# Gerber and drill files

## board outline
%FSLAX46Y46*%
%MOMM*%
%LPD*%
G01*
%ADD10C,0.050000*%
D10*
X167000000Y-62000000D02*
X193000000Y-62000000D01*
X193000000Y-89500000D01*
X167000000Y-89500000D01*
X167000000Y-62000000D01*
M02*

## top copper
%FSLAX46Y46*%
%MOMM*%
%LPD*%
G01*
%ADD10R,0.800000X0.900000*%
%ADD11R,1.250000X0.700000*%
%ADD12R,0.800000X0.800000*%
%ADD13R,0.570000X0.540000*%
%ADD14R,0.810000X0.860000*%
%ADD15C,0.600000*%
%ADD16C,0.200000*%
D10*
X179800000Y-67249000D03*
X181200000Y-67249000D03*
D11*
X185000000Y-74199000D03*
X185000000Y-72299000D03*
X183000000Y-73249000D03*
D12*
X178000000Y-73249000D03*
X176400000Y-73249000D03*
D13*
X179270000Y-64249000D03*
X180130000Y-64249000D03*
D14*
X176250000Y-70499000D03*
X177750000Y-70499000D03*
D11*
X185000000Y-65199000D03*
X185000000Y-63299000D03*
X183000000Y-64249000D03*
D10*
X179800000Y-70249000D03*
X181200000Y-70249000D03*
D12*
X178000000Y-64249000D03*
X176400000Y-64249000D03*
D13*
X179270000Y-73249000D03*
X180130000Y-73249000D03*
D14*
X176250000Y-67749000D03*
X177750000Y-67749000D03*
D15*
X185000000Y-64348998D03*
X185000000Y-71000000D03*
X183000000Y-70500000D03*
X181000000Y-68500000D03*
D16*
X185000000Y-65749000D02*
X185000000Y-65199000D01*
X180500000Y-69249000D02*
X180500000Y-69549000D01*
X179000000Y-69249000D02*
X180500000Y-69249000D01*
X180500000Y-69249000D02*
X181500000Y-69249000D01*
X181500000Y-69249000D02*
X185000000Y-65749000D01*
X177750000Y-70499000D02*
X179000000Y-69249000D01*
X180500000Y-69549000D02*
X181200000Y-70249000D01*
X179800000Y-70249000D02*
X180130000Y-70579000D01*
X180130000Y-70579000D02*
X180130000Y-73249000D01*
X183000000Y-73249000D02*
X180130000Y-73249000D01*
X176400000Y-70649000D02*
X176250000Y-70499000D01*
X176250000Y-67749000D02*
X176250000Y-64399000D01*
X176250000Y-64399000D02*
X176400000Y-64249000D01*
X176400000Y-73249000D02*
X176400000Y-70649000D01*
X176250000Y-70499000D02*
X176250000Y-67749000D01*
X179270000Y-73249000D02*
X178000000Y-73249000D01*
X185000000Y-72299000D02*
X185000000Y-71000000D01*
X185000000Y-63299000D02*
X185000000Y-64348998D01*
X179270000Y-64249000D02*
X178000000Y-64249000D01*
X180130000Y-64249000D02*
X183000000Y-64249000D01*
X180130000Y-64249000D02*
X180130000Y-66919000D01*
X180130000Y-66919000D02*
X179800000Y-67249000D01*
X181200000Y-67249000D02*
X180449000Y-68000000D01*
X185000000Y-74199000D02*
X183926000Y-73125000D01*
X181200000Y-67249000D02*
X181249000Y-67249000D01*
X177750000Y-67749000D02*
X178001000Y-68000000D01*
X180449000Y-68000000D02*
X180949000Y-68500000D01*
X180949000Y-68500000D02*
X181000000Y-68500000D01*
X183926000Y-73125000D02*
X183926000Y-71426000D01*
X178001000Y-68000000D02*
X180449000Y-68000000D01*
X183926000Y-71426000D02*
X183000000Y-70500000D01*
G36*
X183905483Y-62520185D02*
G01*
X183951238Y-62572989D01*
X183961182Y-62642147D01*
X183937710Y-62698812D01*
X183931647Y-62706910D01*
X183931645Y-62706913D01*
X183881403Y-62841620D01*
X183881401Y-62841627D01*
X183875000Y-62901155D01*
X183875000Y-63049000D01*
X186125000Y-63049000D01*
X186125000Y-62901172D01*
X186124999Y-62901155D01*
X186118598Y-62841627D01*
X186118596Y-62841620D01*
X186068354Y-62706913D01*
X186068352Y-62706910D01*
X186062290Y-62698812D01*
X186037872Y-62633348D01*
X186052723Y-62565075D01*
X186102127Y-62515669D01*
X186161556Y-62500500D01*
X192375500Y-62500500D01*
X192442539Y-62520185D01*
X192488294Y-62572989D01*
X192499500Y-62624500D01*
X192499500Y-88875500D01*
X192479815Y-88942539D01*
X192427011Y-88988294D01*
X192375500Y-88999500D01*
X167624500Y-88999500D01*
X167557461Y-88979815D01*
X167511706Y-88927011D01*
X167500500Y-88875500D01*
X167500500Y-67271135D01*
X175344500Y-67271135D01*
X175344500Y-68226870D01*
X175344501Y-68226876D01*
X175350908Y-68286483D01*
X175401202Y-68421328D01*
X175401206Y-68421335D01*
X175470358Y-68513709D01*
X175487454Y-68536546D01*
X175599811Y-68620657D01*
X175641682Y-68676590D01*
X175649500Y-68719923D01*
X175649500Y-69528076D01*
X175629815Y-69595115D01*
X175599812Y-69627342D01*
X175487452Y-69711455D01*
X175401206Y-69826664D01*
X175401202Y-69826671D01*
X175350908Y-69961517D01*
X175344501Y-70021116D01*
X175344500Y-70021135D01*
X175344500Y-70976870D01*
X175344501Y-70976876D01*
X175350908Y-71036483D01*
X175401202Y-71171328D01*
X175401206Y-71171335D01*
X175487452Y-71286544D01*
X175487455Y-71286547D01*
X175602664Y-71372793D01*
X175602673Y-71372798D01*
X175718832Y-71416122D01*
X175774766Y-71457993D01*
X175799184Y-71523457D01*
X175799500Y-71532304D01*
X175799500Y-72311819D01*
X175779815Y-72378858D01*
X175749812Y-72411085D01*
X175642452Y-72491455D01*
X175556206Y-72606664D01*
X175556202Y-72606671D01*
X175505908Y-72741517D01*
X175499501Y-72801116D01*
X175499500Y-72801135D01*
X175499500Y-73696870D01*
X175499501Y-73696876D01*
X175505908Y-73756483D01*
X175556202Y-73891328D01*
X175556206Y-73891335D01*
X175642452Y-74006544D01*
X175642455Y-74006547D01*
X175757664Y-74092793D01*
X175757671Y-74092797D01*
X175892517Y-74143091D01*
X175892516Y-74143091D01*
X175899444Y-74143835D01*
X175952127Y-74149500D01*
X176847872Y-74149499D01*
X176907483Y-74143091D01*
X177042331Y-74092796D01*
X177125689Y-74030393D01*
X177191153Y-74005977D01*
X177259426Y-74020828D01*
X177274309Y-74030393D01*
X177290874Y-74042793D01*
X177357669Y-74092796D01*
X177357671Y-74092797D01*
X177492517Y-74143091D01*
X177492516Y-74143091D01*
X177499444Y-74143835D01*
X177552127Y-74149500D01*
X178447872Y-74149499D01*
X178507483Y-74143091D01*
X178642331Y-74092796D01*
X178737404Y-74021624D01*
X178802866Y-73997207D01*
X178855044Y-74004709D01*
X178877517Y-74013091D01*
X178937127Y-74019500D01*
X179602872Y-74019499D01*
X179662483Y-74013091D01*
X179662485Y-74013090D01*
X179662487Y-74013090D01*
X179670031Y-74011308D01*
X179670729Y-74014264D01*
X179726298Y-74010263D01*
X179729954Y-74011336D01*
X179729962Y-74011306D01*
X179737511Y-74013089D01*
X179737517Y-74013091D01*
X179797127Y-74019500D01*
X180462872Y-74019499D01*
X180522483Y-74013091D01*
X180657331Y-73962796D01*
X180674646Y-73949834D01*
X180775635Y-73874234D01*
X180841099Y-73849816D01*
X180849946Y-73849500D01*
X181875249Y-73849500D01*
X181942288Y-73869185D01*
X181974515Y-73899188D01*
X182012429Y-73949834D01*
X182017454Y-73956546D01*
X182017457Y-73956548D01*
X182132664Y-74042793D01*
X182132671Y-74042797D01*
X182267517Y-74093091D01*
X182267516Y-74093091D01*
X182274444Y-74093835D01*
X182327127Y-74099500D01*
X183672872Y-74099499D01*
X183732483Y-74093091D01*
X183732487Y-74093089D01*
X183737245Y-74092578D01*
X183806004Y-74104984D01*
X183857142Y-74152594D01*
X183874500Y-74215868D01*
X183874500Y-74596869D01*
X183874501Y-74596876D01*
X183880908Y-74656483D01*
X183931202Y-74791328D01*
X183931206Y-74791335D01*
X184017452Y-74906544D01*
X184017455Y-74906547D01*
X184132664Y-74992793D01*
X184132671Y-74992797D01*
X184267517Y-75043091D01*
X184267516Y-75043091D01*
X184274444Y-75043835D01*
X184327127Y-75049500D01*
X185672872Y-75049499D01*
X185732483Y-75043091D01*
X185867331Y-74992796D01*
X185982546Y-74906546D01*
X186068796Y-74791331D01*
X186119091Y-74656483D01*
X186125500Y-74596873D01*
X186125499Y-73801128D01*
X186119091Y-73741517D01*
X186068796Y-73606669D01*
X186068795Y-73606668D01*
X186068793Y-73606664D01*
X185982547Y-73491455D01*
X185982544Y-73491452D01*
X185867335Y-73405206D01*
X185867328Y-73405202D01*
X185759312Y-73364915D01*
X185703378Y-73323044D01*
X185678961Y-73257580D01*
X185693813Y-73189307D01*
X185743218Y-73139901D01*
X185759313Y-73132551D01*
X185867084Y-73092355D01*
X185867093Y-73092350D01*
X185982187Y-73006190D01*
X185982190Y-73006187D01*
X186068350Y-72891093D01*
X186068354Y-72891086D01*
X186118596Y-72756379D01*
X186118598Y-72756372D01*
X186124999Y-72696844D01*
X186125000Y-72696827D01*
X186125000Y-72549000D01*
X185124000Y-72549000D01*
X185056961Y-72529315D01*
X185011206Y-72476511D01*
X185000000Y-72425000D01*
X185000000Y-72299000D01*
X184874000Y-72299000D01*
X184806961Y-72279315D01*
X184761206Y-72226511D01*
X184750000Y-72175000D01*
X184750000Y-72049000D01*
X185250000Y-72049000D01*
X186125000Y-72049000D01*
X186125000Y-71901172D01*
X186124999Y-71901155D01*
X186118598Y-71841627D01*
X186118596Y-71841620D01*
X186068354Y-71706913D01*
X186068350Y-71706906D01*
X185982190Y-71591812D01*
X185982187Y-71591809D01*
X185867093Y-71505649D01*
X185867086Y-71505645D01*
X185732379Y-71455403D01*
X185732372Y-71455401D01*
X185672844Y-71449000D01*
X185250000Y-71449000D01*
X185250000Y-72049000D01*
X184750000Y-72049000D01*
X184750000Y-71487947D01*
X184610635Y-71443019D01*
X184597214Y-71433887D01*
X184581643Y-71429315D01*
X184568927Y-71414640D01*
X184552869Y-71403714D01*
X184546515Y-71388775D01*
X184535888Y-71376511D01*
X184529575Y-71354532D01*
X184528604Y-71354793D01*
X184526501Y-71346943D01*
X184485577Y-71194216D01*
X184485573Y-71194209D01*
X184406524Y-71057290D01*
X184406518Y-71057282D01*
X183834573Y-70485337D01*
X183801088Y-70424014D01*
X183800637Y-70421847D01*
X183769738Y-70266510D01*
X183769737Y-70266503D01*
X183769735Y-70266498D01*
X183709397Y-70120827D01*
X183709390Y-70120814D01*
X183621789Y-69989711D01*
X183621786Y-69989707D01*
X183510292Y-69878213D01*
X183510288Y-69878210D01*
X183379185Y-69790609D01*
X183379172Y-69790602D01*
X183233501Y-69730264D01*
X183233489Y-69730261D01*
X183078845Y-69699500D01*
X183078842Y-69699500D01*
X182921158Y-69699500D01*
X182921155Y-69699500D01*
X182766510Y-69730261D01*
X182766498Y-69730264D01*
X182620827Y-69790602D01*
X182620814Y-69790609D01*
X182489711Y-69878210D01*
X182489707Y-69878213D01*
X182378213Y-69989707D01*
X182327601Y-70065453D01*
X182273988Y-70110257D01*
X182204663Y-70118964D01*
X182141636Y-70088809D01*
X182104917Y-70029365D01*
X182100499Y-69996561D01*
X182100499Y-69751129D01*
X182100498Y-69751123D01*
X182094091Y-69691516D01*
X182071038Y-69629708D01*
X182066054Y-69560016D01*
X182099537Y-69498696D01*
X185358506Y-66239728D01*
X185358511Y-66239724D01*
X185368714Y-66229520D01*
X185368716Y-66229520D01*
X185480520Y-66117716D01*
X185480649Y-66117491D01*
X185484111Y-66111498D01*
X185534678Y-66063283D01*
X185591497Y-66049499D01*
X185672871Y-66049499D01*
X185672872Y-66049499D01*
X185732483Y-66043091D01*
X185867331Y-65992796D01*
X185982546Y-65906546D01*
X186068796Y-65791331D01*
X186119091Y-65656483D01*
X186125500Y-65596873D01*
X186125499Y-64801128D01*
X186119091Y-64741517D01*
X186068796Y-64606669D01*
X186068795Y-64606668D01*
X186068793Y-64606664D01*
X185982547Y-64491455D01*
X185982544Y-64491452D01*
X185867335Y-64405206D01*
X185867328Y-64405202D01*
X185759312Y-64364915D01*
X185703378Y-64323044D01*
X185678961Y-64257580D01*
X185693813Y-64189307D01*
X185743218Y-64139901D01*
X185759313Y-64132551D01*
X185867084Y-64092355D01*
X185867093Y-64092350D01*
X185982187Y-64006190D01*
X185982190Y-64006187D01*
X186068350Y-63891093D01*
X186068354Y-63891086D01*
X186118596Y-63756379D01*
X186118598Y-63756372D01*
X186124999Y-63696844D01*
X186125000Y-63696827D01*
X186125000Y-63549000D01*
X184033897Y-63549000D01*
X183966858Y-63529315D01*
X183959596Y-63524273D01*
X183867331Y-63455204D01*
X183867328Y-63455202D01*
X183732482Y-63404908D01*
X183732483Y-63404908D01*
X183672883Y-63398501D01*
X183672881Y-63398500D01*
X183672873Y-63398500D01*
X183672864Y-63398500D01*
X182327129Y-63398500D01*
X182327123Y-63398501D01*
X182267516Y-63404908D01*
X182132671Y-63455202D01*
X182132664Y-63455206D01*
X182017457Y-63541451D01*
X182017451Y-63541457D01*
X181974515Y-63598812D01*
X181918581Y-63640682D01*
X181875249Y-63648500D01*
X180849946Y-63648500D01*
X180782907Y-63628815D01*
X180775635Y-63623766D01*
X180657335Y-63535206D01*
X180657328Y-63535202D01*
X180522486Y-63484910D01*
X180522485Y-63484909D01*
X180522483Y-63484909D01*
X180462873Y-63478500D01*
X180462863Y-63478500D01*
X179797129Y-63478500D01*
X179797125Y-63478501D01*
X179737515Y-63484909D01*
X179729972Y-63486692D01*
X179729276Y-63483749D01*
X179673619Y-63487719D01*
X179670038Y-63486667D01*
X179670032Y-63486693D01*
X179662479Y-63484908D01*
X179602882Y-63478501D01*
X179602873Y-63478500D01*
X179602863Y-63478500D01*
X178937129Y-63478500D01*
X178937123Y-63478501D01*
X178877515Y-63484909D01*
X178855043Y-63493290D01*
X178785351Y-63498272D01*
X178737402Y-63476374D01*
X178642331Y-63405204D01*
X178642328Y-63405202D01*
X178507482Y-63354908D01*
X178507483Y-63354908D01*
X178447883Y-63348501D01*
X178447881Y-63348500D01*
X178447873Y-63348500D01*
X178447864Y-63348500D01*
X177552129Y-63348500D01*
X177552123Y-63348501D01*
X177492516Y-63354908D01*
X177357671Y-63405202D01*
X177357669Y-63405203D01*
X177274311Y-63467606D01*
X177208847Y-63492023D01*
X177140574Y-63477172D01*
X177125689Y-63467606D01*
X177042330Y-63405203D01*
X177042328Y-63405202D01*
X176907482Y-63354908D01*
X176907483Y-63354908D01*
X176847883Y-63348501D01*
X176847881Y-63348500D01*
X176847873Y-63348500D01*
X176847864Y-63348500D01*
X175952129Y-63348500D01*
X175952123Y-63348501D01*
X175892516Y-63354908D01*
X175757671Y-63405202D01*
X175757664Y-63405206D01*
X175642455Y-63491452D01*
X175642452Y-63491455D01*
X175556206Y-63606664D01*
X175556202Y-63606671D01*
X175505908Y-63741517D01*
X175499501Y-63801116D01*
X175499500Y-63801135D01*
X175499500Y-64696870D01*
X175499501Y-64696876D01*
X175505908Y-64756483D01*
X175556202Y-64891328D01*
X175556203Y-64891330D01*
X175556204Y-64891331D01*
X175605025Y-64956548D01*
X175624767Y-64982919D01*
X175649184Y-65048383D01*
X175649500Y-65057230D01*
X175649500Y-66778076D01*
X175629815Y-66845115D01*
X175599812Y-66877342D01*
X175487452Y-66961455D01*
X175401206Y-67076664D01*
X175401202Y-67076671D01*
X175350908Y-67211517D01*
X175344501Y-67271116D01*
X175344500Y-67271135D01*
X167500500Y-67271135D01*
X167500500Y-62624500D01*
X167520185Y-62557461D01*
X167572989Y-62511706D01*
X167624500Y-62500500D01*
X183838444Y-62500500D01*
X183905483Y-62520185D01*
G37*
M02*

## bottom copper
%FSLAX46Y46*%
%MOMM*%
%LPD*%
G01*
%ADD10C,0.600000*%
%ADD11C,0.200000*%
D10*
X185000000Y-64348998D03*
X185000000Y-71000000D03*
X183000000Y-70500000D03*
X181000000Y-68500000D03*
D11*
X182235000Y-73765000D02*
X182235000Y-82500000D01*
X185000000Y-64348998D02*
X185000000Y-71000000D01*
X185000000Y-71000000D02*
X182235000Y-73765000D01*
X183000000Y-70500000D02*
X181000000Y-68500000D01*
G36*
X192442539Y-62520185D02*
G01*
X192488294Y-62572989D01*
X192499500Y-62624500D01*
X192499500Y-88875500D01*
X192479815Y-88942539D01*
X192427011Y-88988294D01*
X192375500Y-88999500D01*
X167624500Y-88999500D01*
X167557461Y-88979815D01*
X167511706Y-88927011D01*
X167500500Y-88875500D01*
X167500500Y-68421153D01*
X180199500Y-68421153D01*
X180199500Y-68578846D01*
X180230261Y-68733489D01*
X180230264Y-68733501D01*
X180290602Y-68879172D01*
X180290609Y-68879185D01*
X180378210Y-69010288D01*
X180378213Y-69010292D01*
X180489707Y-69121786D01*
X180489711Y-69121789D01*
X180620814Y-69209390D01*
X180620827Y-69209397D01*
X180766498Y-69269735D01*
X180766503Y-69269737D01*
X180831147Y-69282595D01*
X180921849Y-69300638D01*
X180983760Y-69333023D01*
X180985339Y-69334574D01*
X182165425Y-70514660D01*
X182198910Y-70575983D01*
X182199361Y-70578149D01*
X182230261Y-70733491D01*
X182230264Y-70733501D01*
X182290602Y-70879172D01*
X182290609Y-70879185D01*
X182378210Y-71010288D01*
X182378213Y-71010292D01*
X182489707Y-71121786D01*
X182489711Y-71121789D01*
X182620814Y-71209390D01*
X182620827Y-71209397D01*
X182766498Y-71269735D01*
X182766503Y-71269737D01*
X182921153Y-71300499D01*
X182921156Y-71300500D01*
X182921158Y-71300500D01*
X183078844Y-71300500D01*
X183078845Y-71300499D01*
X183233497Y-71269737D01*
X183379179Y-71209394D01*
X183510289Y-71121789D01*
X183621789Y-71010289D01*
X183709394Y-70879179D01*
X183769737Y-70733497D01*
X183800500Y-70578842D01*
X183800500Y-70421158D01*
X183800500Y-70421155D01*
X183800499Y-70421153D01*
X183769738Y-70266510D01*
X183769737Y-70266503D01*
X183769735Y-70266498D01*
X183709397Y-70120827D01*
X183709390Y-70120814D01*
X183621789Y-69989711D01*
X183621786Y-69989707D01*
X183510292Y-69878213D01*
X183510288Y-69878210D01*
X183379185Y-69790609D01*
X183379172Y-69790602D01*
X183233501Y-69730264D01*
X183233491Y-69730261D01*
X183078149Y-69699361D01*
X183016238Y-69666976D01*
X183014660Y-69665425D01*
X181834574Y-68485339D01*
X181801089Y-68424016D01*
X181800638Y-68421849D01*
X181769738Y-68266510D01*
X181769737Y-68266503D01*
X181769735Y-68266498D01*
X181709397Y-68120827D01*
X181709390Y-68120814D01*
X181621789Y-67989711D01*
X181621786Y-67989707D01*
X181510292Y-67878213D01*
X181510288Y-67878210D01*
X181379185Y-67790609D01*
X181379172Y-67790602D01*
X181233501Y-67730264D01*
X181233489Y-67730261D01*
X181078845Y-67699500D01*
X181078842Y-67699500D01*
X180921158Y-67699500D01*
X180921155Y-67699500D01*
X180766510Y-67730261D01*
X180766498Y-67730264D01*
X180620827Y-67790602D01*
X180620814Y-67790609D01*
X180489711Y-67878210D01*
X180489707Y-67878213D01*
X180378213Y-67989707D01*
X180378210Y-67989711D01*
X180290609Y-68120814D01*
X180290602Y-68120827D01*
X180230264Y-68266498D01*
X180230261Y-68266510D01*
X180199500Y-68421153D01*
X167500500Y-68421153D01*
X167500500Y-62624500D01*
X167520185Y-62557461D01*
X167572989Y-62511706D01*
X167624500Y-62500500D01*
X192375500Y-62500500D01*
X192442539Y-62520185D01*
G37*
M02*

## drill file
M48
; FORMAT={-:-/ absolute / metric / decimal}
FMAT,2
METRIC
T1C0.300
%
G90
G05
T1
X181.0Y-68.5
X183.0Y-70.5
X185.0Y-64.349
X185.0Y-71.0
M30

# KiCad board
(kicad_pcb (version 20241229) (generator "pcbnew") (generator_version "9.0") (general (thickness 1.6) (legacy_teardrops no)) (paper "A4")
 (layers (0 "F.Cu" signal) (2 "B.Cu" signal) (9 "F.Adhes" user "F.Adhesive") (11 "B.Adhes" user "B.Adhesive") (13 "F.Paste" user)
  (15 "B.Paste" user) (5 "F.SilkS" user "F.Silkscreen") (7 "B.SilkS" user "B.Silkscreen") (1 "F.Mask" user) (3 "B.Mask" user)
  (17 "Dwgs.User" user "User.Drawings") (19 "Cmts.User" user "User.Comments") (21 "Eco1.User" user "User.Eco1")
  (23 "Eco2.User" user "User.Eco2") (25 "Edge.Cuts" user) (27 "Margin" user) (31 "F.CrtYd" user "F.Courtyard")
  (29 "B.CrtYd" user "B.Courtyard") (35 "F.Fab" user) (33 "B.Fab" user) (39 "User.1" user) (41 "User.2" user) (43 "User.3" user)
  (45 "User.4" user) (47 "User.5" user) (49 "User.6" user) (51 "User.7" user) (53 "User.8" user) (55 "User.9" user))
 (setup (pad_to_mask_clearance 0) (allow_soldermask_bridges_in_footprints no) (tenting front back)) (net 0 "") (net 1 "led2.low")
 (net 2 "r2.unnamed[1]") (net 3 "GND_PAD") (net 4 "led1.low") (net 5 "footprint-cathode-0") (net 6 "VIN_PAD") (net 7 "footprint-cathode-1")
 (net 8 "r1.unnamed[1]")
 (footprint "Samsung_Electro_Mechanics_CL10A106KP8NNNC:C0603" (layer "F.Cu") (at 180.5 67.249 0)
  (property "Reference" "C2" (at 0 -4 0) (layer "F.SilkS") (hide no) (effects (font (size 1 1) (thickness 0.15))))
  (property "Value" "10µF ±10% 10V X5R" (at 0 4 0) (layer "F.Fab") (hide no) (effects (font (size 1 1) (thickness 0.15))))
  (pad "1" smd rect (at -0.7 0 0) (size 0.8 0.9) (layers "F.Cu" "F.Mask" "F.Paste") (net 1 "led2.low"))
  (pad "2" smd rect (at 0.7 0 0) (size 0.8 0.9) (layers "F.Cu" "F.Mask" "F.Paste") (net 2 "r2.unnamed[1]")))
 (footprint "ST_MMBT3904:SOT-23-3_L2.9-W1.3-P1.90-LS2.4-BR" (layer "F.Cu") (at 184 73.249 0)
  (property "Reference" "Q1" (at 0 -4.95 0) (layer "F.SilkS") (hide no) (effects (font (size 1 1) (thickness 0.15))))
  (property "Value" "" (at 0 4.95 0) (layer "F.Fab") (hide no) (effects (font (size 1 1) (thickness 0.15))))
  (pad "1" smd rect (at 1 0.95 0) (size 1.25 0.7) (layers "F.Cu" "F.Mask" "F.Paste") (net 2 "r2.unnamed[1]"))
  (pad "2" smd rect (at 1 -0.95 0) (size 1.25 0.7) (layers "F.Cu" "F.Mask" "F.Paste") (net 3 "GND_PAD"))
  (pad "3" smd rect (at -1 0 0) (size 1.25 0.7) (layers "F.Cu" "F.Mask" "F.Paste") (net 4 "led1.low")))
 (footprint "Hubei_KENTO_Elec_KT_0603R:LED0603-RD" (layer "F.Cu") (at 177.2 73.249 180)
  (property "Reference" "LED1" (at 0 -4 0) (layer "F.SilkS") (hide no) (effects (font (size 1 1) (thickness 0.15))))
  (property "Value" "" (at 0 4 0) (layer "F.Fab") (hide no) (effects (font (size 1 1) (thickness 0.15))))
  (pad "1" smd rect (at -0.8 0 270) (size 0.8 0.8) (layers "F.Cu" "F.Mask" "F.Paste") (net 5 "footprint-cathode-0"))
  (pad "2" smd rect (at 0.8 0 270) (size 0.8 0.8) (layers "F.Cu" "F.Mask" "F.Paste") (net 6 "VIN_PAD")))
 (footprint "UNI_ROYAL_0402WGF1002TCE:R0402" (layer "F.Cu") (at 179.7 64.249 0)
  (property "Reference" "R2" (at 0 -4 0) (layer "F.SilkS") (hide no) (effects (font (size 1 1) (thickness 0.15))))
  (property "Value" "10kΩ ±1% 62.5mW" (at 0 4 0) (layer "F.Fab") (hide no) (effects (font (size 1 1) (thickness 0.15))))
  (pad "1" smd rect (at -0.43 0 0) (size 0.57 0.54) (layers "F.Cu" "F.Mask" "F.Paste") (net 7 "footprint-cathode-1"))
  (pad "2" smd rect (at 0.43 0 0) (size 0.57 0.54) (layers "F.Cu" "F.Mask" "F.Paste") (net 1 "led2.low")))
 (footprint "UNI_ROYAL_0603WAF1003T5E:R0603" (layer "F.Cu") (at 177 70.499 0)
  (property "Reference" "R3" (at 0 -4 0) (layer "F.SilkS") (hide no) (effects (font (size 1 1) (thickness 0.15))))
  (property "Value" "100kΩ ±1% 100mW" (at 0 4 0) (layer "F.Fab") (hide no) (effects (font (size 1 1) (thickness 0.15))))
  (pad "1" smd rect (at -0.75 0 0) (size 0.81 0.86) (layers "F.Cu" "F.Mask" "F.Paste") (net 6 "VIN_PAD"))
  (pad "2" smd rect (at 0.75 0 0) (size 0.81 0.86) (layers "F.Cu" "F.Mask" "F.Paste") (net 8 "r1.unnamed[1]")))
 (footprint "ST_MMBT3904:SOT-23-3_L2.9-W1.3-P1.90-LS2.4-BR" (layer "F.Cu") (at 184 64.249 0)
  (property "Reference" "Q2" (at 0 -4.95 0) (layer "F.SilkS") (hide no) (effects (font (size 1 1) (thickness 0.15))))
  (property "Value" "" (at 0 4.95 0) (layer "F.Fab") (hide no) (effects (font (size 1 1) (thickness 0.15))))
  (pad "1" smd rect (at 1 0.95 0) (size 1.25 0.7) (layers "F.Cu" "F.Mask" "F.Paste") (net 8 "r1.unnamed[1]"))
  (pad "2" smd rect (at 1 -0.95 0) (size 1.25 0.7) (layers "F.Cu" "F.Mask" "F.Paste") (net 3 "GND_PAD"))
  (pad "3" smd rect (at -1 0 0) (size 1.25 0.7) (layers "F.Cu" "F.Mask" "F.Paste") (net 1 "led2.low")))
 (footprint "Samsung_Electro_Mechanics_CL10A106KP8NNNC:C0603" (layer "F.Cu") (at 180.5 70.249 0)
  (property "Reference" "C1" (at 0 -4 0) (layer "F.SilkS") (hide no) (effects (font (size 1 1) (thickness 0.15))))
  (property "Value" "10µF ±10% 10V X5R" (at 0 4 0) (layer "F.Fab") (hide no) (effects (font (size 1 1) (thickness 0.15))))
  (pad "1" smd rect (at -0.7 0 0) (size 0.8 0.9) (layers "F.Cu" "F.Mask" "F.Paste") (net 4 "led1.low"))
  (pad "2" smd rect (at 0.7 0 0) (size 0.8 0.9) (layers "F.Cu" "F.Mask" "F.Paste") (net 8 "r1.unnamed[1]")))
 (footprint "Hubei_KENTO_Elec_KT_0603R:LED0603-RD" (layer "F.Cu") (at 177.2 64.249 180)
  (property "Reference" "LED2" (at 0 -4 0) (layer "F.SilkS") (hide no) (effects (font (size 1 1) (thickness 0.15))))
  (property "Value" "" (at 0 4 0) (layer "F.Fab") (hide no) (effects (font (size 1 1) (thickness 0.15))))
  (pad "1" smd rect (at -0.8 0 270) (size 0.8 0.8) (layers "F.Cu" "F.Mask" "F.Paste") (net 7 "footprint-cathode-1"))
  (pad "2" smd rect (at 0.8 0 270) (size 0.8 0.8) (layers "F.Cu" "F.Mask" "F.Paste") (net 6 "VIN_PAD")))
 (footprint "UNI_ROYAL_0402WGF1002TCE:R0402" (layer "F.Cu") (at 179.7 73.249 0)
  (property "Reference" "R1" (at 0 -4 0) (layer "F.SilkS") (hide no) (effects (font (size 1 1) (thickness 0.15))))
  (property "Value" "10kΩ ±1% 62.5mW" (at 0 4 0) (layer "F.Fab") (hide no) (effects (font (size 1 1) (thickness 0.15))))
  (pad "1" smd rect (at -0.43 0 0) (size 0.57 0.54) (layers "F.Cu" "F.Mask" "F.Paste") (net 5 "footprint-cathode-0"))
  (pad "2" smd rect (at 0.43 0 0) (size 0.57 0.54) (layers "F.Cu" "F.Mask" "F.Paste") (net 4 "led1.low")))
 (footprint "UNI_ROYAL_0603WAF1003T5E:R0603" (layer "F.Cu") (at 177 67.749 0)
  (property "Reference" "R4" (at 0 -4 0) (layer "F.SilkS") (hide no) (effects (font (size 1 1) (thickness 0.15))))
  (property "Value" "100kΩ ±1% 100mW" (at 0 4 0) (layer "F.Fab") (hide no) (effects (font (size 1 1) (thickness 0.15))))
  (pad "1" smd rect (at -0.75 0 0) (size 0.81 0.86) (layers "F.Cu" "F.Mask" "F.Paste") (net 6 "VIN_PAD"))
  (pad "2" smd rect (at 0.75 0 0) (size 0.81 0.86) (layers "F.Cu" "F.Mask" "F.Paste") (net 2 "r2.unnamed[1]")))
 (via (at 185 64.348998) (size 0.6) (drill 0.3) (layers "F.Cu" "B.Cu") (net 3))
 (via (at 185 71) (size 0.6) (drill 0.3) (layers "F.Cu" "B.Cu") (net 3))
 (via (at 183 70.5) (size 0.6) (drill 0.3) (layers "F.Cu" "B.Cu") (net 2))
 (via (at 181 68.5) (size 0.6) (drill 0.3) (layers "F.Cu" "B.Cu") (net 2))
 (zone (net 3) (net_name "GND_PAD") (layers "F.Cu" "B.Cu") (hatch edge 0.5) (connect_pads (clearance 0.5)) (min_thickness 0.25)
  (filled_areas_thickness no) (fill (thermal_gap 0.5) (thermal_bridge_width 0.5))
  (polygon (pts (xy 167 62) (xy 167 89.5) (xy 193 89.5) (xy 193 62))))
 (segment (start 185 65.749) (end 185 65.199) (width 0.2) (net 8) (layer "F.Cu"))
 (segment (start 180.5 69.249) (end 180.5 69.549) (width 0.2) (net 8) (layer "F.Cu"))
 (segment (start 179 69.249) (end 180.5 69.249) (width 0.2) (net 8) (layer "F.Cu"))
 (segment (start 180.5 69.249) (end 181.5 69.249) (width 0.2) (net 8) (layer "F.Cu"))
 (segment (start 181.5 69.249) (end 185 65.749) (width 0.2) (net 8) (layer "F.Cu"))
 (segment (start 177.75 70.499) (end 179 69.249) (width 0.2) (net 8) (layer "F.Cu"))
 (segment (start 180.5 69.549) (end 181.2 70.249) (width 0.2) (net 8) (layer "F.Cu"))
 (segment (start 179.8 70.249) (end 180.13 70.579) (width 0.2) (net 4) (layer "F.Cu"))
 (segment (start 180.13 70.579) (end 180.13 73.249) (width 0.2) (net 4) (layer "F.Cu"))
 (segment (start 183 73.249) (end 180.13 73.249) (width 0.2) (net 4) (layer "F.Cu"))
 (segment (start 176.4 70.649) (end 176.25 70.499) (width 0.2) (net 6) (layer "F.Cu"))
 (segment (start 176.25 67.749) (end 176.25 64.399) (width 0.2) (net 6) (layer "F.Cu"))
 (segment (start 176.25 64.399) (end 176.4 64.249) (width 0.2) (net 6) (layer "F.Cu"))
 (segment (start 176.4 73.249) (end 176.4 70.649) (width 0.2) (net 6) (layer "F.Cu"))
 (segment (start 176.25 70.499) (end 176.25 67.749) (width 0.2) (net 6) (layer "F.Cu"))
 (segment (start 179.27 73.249) (end 178 73.249) (width 0.2) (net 5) (layer "F.Cu"))
 (segment (start 185 72.299) (end 185 71) (width 0.2) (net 3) (layer "F.Cu"))
 (segment (start 185 63.299) (end 185 64.348998) (width 0.2) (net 3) (layer "F.Cu"))
 (segment (start 182.235 73.765) (end 182.235 82.5) (width 0.2) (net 3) (layer "B.Cu"))
 (segment (start 185 64.348998) (end 185 71) (width 0.2) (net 3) (layer "B.Cu"))
 (segment (start 185 71) (end 182.235 73.765) (width 0.2) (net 3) (layer "B.Cu"))
 (segment (start 179.27 64.249) (end 178 64.249) (width 0.2) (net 7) (layer "F.Cu"))
 (segment (start 180.13 64.249) (end 183 64.249) (width 0.2) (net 1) (layer "F.Cu"))
 (segment (start 180.13 64.249) (end 180.13 66.919) (width 0.2) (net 1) (layer "F.Cu"))
 (segment (start 180.13 66.919) (end 179.8 67.249) (width 0.2) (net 1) (layer "F.Cu"))
 (segment (start 181.2 67.249) (end 180.449 68) (width 0.2) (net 2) (layer "F.Cu"))
 (segment (start 185 74.199) (end 183.926 73.125) (width 0.2) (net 2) (layer "F.Cu"))
 (segment (start 181.2 67.249) (end 181.249 67.249) (width 0.2) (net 2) (layer "F.Cu"))
 (segment (start 177.75 67.749) (end 178.001 68) (width 0.2) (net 2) (layer "F.Cu"))
 (segment (start 180.449 68) (end 180.949 68.5) (width 0.2) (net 2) (layer "F.Cu"))
 (segment (start 180.949 68.5) (end 181 68.5) (width 0.2) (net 2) (layer "F.Cu"))
 (segment (start 183.926 73.125) (end 183.926 71.426) (width 0.2) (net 2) (layer "F.Cu"))
 (segment (start 178.001 68) (end 180.449 68) (width 0.2) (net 2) (layer "F.Cu"))
 (segment (start 183.926 71.426) (end 183 70.5) (width 0.2) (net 2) (layer "F.Cu"))
 (segment (start 183 70.5) (end 181 68.5) (width 0.2) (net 2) (layer "B.Cu"))
 (gr_rect (start 167 62) (end 193 89.5) (stroke (width 0.05) (type default)) (fill no) (layer "Edge.Cuts")))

